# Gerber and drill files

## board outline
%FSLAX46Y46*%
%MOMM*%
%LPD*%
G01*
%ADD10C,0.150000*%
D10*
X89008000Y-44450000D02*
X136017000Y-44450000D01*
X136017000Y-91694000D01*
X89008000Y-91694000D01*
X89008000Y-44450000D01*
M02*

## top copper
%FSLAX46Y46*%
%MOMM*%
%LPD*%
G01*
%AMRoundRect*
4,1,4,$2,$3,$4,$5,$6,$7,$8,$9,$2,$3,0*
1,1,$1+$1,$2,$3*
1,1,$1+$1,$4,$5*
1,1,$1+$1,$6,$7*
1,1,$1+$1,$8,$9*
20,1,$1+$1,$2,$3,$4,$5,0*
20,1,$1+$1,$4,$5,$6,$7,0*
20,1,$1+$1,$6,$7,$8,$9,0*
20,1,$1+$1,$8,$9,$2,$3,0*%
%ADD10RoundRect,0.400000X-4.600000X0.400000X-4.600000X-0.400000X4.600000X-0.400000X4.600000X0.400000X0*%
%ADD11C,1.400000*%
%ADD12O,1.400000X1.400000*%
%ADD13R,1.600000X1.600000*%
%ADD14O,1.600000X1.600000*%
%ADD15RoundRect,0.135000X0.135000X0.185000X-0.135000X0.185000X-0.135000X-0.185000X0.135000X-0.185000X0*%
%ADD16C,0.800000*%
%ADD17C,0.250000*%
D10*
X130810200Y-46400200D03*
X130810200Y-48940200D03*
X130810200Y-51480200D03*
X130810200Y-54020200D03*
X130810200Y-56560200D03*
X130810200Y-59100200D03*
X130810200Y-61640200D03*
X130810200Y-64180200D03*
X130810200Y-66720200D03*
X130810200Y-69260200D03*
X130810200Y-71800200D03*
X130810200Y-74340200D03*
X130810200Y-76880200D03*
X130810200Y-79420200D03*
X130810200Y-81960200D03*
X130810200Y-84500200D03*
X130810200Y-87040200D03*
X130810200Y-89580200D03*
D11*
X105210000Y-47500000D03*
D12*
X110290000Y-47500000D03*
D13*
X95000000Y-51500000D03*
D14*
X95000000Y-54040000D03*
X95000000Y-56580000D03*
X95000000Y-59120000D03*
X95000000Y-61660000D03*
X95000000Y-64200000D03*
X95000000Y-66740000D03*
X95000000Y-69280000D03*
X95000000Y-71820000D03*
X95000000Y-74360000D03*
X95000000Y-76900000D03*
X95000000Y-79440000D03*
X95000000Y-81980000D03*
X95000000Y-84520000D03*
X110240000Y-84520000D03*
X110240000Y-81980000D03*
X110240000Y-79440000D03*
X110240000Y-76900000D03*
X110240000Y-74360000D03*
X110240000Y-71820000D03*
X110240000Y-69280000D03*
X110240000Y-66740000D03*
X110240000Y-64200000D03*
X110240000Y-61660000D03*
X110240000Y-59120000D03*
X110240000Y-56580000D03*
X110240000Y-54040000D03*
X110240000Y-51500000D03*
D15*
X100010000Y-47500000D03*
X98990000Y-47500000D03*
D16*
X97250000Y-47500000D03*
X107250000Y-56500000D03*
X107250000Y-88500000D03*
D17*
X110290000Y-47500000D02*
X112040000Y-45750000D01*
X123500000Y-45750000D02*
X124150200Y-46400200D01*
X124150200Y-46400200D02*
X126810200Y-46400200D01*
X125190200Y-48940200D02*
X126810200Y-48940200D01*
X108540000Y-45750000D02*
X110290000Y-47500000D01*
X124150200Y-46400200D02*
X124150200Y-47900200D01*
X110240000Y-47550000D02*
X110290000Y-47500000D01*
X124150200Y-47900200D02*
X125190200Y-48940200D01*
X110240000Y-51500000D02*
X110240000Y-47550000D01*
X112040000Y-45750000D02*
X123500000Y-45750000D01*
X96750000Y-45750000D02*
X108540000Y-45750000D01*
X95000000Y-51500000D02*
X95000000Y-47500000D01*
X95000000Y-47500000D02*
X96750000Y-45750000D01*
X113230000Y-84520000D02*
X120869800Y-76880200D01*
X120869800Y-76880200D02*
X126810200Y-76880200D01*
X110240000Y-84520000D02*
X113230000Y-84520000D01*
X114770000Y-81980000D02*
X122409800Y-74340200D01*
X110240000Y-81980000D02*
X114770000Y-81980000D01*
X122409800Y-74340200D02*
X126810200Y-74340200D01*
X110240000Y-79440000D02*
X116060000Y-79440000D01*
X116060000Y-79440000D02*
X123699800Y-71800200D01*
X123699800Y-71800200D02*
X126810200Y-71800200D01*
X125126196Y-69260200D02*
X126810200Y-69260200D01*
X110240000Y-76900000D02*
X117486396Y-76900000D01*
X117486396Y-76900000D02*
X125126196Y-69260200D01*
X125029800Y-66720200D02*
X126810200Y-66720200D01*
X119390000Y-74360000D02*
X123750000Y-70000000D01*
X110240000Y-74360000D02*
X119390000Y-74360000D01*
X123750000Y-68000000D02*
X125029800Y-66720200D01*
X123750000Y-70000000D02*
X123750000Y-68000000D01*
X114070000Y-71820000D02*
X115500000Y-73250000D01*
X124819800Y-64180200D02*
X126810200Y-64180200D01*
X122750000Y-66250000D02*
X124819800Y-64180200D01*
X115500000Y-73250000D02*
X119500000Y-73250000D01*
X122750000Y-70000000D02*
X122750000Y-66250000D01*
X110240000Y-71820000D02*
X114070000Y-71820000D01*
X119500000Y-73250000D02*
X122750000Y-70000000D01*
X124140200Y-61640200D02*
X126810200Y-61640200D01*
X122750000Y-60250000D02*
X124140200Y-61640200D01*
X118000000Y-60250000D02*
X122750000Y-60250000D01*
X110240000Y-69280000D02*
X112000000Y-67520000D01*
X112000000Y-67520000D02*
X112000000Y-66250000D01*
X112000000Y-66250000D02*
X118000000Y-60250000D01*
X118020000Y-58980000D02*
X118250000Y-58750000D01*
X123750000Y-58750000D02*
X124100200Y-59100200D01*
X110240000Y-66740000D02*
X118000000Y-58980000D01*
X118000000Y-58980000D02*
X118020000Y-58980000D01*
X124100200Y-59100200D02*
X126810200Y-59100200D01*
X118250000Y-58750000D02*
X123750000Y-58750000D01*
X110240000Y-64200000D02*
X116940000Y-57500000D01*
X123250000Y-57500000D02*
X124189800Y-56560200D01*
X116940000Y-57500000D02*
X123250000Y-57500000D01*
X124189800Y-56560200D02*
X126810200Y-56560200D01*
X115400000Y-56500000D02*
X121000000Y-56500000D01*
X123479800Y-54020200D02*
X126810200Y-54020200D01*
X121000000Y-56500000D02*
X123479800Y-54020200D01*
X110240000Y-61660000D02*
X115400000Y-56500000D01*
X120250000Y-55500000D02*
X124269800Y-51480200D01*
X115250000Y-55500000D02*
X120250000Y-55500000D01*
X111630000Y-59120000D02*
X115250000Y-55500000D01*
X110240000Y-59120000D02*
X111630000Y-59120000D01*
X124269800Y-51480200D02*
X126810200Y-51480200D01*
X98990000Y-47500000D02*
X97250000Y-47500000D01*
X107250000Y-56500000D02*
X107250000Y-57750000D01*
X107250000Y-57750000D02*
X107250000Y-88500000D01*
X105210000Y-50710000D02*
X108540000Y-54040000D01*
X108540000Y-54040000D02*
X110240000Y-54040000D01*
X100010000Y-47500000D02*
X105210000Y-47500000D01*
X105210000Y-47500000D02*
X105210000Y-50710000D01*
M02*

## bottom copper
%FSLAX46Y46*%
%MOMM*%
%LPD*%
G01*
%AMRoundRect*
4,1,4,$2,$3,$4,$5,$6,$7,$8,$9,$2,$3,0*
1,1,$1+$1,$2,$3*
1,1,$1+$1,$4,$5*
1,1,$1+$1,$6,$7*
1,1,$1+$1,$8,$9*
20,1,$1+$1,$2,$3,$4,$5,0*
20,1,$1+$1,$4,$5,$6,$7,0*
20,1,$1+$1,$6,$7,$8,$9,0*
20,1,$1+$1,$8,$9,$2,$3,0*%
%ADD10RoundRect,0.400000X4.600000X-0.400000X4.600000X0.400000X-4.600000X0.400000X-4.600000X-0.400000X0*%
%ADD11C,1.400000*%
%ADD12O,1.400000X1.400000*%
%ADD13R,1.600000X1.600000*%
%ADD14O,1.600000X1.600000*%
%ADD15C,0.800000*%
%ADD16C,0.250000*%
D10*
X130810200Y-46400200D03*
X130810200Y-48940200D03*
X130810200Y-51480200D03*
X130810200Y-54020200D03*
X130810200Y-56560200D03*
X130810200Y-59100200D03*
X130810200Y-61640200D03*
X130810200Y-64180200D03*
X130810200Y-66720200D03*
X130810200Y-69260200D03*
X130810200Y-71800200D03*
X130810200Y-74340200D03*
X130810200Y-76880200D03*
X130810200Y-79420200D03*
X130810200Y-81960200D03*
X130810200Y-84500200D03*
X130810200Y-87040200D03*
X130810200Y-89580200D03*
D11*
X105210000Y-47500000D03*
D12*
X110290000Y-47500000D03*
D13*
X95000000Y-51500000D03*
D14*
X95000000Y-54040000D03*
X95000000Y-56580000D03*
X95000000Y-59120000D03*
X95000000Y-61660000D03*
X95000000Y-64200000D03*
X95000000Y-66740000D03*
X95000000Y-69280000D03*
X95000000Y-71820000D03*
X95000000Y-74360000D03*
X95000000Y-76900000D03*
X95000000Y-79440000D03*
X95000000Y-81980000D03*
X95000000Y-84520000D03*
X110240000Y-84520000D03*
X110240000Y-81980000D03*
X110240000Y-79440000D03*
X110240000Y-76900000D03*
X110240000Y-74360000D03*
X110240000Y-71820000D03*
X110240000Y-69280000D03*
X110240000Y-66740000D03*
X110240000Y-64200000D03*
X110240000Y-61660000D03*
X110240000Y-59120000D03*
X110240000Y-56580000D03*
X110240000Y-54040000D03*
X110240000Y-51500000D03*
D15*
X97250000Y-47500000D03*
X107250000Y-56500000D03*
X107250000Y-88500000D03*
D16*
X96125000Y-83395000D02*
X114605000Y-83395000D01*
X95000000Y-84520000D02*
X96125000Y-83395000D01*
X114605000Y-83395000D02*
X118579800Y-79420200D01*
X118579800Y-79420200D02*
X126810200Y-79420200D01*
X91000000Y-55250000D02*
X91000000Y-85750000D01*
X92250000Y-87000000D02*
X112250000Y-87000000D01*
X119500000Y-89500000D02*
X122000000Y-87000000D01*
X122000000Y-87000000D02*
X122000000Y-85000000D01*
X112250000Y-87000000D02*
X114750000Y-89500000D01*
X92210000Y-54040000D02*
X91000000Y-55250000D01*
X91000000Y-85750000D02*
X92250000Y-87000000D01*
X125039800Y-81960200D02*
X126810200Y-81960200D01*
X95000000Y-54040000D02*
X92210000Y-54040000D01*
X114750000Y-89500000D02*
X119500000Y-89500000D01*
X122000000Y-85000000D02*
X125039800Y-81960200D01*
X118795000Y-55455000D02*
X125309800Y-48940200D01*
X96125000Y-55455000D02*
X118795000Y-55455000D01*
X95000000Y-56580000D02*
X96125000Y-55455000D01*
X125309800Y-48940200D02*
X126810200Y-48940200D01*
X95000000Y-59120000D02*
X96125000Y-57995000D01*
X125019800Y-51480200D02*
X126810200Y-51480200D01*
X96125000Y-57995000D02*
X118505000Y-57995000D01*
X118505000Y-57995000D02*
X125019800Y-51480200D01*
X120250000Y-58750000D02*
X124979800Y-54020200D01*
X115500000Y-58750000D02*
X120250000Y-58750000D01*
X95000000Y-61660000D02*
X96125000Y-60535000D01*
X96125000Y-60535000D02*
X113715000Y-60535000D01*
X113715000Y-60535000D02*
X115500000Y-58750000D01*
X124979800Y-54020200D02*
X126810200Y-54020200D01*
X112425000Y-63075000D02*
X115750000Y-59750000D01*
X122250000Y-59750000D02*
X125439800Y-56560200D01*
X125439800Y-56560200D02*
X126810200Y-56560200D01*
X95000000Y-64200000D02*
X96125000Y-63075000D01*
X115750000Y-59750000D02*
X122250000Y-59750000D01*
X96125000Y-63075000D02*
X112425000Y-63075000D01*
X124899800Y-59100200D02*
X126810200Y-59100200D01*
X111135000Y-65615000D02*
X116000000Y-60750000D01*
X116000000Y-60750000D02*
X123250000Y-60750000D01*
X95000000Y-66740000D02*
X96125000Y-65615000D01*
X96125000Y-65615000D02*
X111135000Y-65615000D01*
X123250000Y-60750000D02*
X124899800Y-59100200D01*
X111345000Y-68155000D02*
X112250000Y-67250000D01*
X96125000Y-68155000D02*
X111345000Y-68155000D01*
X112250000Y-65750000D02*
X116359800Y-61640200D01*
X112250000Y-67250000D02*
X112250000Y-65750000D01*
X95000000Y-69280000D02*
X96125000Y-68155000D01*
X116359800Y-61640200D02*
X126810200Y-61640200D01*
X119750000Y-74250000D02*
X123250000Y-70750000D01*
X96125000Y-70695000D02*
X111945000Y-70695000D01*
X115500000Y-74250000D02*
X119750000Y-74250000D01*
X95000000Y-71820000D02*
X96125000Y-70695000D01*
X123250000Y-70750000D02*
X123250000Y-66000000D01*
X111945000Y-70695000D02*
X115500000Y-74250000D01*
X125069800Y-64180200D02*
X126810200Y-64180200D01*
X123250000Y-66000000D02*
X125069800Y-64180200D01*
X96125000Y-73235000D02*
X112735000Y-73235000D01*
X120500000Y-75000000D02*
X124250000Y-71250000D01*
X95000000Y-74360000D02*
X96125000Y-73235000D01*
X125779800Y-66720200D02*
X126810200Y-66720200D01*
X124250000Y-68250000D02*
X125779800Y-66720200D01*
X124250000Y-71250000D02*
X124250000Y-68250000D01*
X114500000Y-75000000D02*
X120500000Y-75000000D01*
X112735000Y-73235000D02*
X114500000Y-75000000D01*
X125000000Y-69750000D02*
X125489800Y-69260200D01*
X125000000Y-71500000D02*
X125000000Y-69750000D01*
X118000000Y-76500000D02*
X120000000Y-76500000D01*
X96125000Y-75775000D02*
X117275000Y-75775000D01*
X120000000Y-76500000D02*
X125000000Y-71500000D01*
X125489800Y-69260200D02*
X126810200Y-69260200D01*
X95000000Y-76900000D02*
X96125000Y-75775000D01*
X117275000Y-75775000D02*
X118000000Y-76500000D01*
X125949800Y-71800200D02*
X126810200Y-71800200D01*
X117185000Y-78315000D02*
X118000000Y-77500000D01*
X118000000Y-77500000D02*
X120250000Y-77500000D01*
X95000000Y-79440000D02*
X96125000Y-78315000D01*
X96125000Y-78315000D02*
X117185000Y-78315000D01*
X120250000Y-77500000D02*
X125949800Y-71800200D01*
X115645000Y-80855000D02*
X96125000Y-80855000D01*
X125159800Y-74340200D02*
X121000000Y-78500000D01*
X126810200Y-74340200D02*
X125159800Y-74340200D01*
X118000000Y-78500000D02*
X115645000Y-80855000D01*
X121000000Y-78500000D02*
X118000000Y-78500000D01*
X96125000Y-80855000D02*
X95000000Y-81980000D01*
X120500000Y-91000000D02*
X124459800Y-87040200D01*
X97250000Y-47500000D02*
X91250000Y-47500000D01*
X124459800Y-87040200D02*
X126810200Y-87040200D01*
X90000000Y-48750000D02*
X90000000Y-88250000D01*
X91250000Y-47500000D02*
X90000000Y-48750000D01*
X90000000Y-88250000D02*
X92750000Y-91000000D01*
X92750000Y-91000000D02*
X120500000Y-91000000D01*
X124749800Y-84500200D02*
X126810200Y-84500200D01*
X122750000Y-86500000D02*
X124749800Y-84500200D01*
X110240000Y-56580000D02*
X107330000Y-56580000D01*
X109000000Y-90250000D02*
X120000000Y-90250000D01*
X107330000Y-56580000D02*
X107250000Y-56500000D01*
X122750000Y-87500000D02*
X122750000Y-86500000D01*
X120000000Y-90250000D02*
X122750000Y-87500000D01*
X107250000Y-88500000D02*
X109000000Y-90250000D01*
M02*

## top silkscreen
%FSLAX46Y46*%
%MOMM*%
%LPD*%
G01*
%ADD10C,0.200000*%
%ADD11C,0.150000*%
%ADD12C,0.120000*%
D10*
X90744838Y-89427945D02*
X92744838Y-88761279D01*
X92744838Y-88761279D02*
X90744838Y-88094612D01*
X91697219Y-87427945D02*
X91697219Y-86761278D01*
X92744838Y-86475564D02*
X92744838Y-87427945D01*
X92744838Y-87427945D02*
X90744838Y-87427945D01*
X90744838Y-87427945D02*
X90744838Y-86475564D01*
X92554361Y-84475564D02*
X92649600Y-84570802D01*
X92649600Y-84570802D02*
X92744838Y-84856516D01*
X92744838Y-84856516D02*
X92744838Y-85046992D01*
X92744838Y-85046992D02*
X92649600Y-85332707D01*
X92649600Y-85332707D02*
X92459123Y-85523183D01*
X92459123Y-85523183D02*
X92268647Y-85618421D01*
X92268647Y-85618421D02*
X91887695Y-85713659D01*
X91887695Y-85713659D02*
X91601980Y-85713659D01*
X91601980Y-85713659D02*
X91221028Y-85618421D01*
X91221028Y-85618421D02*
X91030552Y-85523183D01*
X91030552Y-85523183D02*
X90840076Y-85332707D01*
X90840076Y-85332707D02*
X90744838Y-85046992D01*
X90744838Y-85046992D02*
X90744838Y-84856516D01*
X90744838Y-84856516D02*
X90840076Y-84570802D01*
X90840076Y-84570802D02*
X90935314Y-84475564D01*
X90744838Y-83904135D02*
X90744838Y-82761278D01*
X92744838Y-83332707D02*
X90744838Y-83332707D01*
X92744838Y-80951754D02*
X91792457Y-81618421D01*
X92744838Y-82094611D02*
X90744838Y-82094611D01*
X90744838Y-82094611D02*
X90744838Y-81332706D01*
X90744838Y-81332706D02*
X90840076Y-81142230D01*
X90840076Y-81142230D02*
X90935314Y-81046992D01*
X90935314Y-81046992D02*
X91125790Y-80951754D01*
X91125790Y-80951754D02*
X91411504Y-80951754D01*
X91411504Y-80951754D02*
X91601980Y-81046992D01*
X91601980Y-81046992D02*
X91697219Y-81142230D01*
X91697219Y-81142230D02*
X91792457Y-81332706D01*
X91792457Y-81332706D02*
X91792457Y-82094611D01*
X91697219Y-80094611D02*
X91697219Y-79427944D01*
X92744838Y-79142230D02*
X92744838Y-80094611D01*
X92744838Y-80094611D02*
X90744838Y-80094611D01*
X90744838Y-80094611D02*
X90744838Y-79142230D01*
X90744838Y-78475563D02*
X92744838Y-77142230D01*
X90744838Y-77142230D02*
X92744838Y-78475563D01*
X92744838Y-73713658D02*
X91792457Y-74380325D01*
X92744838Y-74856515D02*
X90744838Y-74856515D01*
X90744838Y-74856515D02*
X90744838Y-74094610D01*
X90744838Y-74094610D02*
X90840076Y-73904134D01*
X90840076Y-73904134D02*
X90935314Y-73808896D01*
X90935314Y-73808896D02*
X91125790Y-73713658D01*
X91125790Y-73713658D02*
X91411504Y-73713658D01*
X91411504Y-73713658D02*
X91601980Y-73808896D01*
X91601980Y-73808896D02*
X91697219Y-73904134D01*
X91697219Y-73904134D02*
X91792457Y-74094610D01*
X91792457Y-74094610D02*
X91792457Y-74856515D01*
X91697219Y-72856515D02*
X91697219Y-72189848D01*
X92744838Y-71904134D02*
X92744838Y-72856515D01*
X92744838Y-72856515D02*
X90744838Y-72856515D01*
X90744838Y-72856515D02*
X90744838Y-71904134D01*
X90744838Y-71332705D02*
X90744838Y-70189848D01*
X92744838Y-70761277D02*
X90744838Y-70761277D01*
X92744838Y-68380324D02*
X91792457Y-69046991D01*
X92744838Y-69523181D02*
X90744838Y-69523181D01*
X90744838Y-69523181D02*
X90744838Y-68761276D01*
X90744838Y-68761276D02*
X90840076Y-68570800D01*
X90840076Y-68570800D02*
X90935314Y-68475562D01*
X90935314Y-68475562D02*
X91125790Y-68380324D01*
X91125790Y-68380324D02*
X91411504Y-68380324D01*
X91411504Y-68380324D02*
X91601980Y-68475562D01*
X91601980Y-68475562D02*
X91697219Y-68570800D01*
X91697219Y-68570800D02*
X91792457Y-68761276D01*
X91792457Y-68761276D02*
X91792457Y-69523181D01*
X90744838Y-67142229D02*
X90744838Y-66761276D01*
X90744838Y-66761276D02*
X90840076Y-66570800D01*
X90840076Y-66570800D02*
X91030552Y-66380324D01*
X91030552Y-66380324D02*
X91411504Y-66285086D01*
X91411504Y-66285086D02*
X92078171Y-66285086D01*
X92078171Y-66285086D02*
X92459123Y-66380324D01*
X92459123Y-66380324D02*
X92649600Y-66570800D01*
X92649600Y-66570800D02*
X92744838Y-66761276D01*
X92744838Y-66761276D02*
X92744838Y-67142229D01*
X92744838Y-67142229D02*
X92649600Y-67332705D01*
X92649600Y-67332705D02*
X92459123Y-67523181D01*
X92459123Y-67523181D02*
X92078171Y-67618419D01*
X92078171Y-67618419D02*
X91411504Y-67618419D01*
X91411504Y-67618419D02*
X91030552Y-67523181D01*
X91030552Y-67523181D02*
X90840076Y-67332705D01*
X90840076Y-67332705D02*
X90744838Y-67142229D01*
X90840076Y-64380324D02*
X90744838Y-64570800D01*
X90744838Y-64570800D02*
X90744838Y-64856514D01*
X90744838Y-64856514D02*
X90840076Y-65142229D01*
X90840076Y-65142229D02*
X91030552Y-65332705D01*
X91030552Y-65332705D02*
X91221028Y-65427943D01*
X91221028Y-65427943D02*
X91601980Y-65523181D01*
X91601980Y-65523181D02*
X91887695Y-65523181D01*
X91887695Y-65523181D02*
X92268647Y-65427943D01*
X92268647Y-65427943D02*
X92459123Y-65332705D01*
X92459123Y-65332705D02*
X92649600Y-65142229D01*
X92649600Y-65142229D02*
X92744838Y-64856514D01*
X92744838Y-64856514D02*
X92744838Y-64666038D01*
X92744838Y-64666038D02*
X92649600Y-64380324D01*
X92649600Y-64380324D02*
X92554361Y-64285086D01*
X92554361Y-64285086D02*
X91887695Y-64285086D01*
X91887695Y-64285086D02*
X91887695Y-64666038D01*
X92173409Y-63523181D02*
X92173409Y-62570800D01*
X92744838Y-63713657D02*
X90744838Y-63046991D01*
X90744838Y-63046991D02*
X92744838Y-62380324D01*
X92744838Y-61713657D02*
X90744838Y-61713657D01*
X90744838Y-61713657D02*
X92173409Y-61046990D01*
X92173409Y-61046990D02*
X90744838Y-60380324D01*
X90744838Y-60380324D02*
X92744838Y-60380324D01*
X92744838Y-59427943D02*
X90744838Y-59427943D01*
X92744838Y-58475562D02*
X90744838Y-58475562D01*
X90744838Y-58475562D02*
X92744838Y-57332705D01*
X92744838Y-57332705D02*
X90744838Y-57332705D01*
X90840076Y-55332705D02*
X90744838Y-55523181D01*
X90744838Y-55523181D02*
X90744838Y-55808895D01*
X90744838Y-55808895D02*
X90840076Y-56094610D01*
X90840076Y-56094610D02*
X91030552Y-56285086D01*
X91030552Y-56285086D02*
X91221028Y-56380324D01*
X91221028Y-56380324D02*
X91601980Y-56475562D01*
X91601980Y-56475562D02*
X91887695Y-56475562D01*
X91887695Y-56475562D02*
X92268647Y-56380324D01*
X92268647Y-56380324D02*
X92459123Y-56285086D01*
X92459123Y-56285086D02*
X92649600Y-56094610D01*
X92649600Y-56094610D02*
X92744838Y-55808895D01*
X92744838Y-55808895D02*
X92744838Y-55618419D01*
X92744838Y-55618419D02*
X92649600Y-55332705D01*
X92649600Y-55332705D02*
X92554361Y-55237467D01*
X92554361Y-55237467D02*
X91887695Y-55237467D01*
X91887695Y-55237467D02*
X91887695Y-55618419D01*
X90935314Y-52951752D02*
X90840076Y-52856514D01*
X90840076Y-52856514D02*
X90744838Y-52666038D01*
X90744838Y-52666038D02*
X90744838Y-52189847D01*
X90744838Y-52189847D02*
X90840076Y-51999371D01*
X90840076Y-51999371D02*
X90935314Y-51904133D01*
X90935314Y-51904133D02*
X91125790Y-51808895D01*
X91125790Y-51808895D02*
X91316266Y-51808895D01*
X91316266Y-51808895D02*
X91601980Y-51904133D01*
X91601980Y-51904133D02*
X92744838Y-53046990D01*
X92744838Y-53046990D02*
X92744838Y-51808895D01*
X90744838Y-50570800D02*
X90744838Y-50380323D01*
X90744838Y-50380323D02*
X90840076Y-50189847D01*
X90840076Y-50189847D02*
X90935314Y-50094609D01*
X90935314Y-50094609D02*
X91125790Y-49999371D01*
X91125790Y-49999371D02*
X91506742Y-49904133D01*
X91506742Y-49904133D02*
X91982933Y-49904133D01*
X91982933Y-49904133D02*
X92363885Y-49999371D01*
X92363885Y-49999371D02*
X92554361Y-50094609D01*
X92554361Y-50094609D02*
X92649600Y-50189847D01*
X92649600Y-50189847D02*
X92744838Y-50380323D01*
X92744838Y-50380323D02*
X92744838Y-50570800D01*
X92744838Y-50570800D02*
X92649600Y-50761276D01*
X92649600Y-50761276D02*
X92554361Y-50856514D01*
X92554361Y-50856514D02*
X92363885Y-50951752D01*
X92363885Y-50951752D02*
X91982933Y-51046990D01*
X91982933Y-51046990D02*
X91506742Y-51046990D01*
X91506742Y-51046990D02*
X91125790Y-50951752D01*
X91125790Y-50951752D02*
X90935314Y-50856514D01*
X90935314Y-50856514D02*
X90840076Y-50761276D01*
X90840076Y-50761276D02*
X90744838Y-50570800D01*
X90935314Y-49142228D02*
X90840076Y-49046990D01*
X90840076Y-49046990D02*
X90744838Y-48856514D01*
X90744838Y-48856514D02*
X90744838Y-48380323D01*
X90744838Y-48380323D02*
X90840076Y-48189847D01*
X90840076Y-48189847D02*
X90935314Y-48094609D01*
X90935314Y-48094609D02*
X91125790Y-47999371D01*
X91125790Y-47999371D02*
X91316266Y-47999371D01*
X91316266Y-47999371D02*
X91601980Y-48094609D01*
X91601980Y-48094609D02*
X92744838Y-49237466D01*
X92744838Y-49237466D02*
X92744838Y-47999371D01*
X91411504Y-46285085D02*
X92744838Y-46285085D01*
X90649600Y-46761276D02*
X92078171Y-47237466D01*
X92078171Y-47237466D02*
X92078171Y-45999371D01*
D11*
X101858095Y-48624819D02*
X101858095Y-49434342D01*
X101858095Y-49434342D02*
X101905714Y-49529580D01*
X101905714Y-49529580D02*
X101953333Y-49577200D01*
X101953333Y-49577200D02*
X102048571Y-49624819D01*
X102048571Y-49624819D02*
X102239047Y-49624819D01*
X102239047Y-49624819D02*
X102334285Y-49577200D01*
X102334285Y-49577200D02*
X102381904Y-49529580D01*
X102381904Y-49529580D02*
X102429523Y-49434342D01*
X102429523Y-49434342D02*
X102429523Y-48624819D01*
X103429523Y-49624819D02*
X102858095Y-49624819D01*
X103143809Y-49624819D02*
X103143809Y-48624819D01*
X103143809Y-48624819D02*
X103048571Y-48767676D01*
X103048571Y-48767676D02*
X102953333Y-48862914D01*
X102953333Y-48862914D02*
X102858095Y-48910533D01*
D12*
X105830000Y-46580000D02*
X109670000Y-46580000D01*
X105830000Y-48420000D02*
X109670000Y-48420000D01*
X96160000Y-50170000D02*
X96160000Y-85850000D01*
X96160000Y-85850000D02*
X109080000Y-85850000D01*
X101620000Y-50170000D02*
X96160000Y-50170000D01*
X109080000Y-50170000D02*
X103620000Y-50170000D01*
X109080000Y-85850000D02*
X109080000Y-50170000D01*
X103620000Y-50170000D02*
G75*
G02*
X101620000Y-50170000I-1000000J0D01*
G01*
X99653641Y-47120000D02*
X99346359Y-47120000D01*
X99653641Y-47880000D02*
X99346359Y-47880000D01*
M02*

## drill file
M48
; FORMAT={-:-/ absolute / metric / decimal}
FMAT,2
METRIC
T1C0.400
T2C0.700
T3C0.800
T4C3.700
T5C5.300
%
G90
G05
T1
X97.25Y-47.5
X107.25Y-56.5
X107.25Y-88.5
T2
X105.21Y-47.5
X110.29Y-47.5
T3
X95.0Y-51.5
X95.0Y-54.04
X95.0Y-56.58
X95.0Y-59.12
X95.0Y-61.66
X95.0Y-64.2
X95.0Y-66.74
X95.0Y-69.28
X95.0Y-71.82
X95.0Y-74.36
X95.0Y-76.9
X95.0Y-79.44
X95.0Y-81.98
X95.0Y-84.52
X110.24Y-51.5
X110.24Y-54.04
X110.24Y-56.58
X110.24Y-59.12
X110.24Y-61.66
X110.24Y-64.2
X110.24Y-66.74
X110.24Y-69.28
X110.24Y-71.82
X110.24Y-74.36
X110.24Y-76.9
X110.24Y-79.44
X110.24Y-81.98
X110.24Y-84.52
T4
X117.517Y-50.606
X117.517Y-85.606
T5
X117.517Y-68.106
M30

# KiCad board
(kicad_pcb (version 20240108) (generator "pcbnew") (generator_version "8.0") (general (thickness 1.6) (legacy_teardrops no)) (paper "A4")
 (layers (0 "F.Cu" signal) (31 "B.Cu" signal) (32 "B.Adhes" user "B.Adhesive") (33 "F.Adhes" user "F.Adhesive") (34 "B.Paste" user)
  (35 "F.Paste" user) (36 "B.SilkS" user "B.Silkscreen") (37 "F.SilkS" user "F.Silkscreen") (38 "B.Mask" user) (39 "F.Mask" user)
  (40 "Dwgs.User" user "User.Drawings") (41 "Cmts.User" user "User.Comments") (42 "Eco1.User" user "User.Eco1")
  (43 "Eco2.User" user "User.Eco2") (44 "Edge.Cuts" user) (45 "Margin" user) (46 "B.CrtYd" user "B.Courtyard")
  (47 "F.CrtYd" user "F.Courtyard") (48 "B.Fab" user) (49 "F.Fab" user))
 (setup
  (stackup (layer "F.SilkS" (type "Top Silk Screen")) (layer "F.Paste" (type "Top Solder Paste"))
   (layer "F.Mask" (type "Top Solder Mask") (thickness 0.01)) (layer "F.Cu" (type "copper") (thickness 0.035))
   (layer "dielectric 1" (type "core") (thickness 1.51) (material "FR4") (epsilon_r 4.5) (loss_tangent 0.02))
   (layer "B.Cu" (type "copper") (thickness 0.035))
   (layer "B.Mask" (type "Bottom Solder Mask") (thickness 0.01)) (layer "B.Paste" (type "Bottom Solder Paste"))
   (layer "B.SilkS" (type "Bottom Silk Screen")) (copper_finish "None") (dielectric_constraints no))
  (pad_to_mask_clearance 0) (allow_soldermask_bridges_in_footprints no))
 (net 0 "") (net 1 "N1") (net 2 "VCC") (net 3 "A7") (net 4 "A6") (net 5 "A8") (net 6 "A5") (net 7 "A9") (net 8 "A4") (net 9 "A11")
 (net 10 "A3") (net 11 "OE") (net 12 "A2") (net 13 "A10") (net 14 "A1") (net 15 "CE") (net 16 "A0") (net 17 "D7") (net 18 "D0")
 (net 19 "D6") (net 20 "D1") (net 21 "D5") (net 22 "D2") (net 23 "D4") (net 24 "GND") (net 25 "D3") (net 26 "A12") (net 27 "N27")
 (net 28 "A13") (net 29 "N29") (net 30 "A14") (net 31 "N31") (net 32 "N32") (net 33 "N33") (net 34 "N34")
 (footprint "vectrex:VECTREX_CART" (layer "F.Cu") (at 130.8102 67.9902 -90)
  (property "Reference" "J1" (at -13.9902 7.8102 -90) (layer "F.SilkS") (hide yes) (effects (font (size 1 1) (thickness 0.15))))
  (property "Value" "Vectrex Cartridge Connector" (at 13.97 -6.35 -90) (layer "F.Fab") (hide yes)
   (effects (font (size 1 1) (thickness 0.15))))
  (pad "1" connect roundrect (at -21.59 4 90) (size 1.6 10) (drill (offset 0 4)) (layers "B.Cu" "B.Mask") (roundrect_rratio 0.25)
   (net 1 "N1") (zone_connect 2))
  (pad "2" connect roundrect (at -21.59 4 270) (size 1.6 10) (drill (offset 0 -4)) (layers "F.Cu" "F.Mask") (roundrect_rratio 0.25)
   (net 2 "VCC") (zone_connect 2))
  (pad "3" connect roundrect (at -19.05 4 90) (size 1.6 10) (drill (offset 0 4)) (layers "B.Cu" "B.Mask") (roundrect_rratio 0.25)
   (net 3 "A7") (zone_connect 2))
  (pad "4" connect roundrect (at -19.05 4 270) (size 1.6 10) (drill (offset 0 -4)) (layers "F.Cu" "F.Mask") (roundrect_rratio 0.25)
   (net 2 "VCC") (zone_connect 2))
  (pad "5" connect roundrect (at -16.51 4 90) (size 1.6 10) (drill (offset 0 4)) (layers "B.Cu" "B.Mask") (roundrect_rratio 0.25)
   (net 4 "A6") (zone_connect 2))
  (pad "6" connect roundrect (at -16.51 4 270) (size 1.6 10) (drill (offset 0 -4)) (layers "F.Cu" "F.Mask") (roundrect_rratio 0.25)
   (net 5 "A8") (zone_connect 2))
  (pad "7" connect roundrect (at -13.97 4 90) (size 1.6 10) (drill (offset 0 4)) (layers "B.Cu" "B.Mask") (roundrect_rratio 0.25)
   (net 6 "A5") (zone_connect 2))
  (pad "8" connect roundrect (at -13.97 4 270) (size 1.6 10) (drill (offset 0 -4)) (layers "F.Cu" "F.Mask") (roundrect_rratio 0.25)
   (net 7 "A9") (zone_connect 2))
  (pad "9" connect roundrect (at -11.43 4 90) (size 1.6 10) (drill (offset 0 4)) (layers "B.Cu" "B.Mask") (roundrect_rratio 0.25)
   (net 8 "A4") (zone_connect 2))
  (pad "10" connect roundrect (at -11.43 4 270) (size 1.6 10) (drill (offset 0 -4)) (layers "F.Cu" "F.Mask") (roundrect_rratio 0.25)
   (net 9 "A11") (zone_connect 2))
  (pad "11" connect roundrect (at -8.89 4 90) (size 1.6 10) (drill (offset 0 4)) (layers "B.Cu" "B.Mask") (roundrect_rratio 0.25)
   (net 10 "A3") (zone_connect 2))
  (pad "12" connect roundrect (at -8.89 4 270) (size 1.6 10) (drill (offset 0 -4)) (layers "F.Cu" "F.Mask") (roundrect_rratio 0.25)
   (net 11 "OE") (zone_connect 2))
  (pad "13" connect roundrect (at -6.35 4 90) (size 1.6 10) (drill (offset 0 4)) (layers "B.Cu" "B.Mask") (roundrect_rratio 0.25)
   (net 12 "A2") (zone_connect 2))
  (pad "14" connect roundrect (at -6.35 4 270) (size 1.6 10) (drill (offset 0 -4)) (layers "F.Cu" "F.Mask") (roundrect_rratio 0.25)
   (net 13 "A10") (zone_connect 2))
  (pad "15" connect roundrect (at -3.81 4 90) (size 1.6 10) (drill (offset 0 4)) (layers "B.Cu" "B.Mask") (roundrect_rratio 0.25)
   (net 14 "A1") (zone_connect 2))
  (pad "16" connect roundrect (at -3.81 4 270) (size 1.6 10) (drill (offset 0 -4)) (layers "F.Cu" "F.Mask") (roundrect_rratio 0.25)
   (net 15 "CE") (zone_connect 2))
  (pad "17" connect roundrect (at -1.27 4 90) (size 1.6 10) (drill (offset 0 4)) (layers "B.Cu" "B.Mask") (roundrect_rratio 0.25)
   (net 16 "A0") (zone_connect 2))
  (pad "18" connect roundrect (at -1.27 4 270) (size 1.6 10) (drill (offset 0 -4)) (layers "F.Cu" "F.Mask") (roundrect_rratio 0.25)
   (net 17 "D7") (zone_connect 2))
  (pad "19" connect roundrect (at 1.27 4 90) (size 1.6 10) (drill (offset 0 4)) (layers "B.Cu" "B.Mask") (roundrect_rratio 0.25)
   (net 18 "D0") (zone_connect 2))
  (pad "20" connect roundrect (at 1.27 4 270) (size 1.6 10) (drill (offset 0 -4)) (layers "F.Cu" "F.Mask") (roundrect_rratio 0.25)
   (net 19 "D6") (zone_connect 2))
  (pad "21" connect roundrect (at 3.81 4 90) (size 1.6 10) (drill (offset 0 4)) (layers "B.Cu" "B.Mask") (roundrect_rratio 0.25)
   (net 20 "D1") (zone_connect 2))
  (pad "22" connect roundrect (at 3.81 4 270) (size 1.6 10) (drill (offset 0 -4)) (layers "F.Cu" "F.Mask") (roundrect_rratio 0.25)
   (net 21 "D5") (zone_connect 2))
  (pad "23" connect roundrect (at 6.35 4 90) (size 1.6 10) (drill (offset 0 4)) (layers "B.Cu" "B.Mask") (roundrect_rratio 0.25)
   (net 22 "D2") (zone_connect 2))
  (pad "24" connect roundrect (at 6.35 4 270) (size 1.6 10) (drill (offset 0 -4)) (layers "F.Cu" "F.Mask") (roundrect_rratio 0.25)
   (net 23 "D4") (zone_connect 2))
  (pad "25" connect roundrect (at 8.89 4 90) (size 1.6 10) (drill (offset 0 4)) (layers "B.Cu" "B.Mask") (roundrect_rratio 0.25)
   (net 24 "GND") (zone_connect 2))
  (pad "26" connect roundrect (at 8.89 4 270) (size 1.6 10) (drill (offset 0 -4)) (layers "F.Cu" "F.Mask") (roundrect_rratio 0.25)
   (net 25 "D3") (zone_connect 2))
  (pad "27" connect roundrect (at 11.43 4 90) (size 1.6 10) (drill (offset 0 4)) (layers "B.Cu" "B.Mask") (roundrect_rratio 0.25)
   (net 24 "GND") (zone_connect 2))
  (pad "28" connect roundrect (at 11.43 4 270) (size 1.6 10) (drill (offset 0 -4)) (layers "F.Cu" "F.Mask") (roundrect_rratio 0.25)
   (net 24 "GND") (zone_connect 2))
  (pad "29" connect roundrect (at 13.97 4 90) (size 1.6 10) (drill (offset 0 4)) (layers "B.Cu" "B.Mask") (roundrect_rratio 0.25)
   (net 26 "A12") (zone_connect 2))
  (pad "30" connect roundrect (at 13.97 4 270) (size 1.6 10) (drill (offset 0 -4)) (layers "F.Cu" "F.Mask") (roundrect_rratio 0.25)
   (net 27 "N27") (zone_connect 2))
  (pad "31" connect roundrect (at 16.51 4 90) (size 1.6 10) (drill (offset 0 4)) (layers "B.Cu" "B.Mask") (roundrect_rratio 0.25)
   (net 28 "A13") (zone_connect 2))
  (pad "32" connect roundrect (at 16.51 4 270) (size 1.6 10) (drill (offset 0 -4)) (layers "F.Cu" "F.Mask") (roundrect_rratio 0.25)
   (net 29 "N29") (zone_connect 2))
  (pad "33" connect roundrect (at 19.05 4 90) (size 1.6 10) (drill (offset 0 4)) (layers "B.Cu" "B.Mask") (roundrect_rratio 0.25)
   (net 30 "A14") (zone_connect 2))
  (pad "34" connect roundrect (at 19.05 4 270) (size 1.6 10) (drill (offset 0 -4)) (layers "F.Cu" "F.Mask") (roundrect_rratio 0.25)
   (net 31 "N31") (zone_connect 2))
  (pad "35" connect roundrect (at 21.59 4 90) (size 1.6 10) (drill (offset 0 4)) (layers "B.Cu" "B.Mask") (roundrect_rratio 0.25)
   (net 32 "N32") (zone_connect 2))
  (pad "36" connect roundrect (at 21.59 4 270) (size 1.6 10) (drill (offset 0 -4)) (layers "F.Cu" "F.Mask") (roundrect_rratio 0.25)
   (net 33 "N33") (zone_connect 2)))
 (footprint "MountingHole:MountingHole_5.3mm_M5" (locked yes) (layer "F.Cu") (at 117.5172 68.1056)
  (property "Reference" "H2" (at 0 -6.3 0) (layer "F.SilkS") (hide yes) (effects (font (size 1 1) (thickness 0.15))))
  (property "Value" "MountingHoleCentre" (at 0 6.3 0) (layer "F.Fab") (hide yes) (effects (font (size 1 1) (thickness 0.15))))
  (pad "" np_thru_hole circle (at 0 0) (size 5.3 5.3) (drill 5.3) (layers "*.Cu" "*.Mask")))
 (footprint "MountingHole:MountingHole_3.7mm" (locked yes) (layer "F.Cu") (at 117.5172 50.6056)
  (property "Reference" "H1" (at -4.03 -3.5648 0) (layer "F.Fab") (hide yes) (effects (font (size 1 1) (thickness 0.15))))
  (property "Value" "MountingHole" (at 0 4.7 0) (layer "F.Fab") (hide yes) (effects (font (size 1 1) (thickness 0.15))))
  (pad "" np_thru_hole circle (at 0 0) (size 3.7 3.7) (drill 3.7) (layers "*.Cu" "*.Mask")))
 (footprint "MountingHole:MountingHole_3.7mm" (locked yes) (layer "F.Cu") (at 117.5172 85.6056)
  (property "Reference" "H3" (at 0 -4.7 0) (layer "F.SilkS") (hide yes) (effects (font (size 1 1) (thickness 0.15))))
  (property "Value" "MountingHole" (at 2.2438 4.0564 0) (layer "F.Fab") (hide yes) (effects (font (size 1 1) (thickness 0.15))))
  (pad "" np_thru_hole circle (at 0 0) (size 3.7 3.7) (drill 3.7) (layers "*.Cu" "*.Mask")))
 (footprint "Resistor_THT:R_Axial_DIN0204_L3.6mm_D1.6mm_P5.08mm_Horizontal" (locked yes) (layer "F.Cu") (at 105.21 47.5)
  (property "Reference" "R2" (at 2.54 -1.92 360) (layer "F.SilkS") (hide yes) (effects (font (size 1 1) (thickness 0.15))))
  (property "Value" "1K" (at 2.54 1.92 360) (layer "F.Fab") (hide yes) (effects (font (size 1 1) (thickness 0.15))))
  (fp_line (start 0.62 -0.92) (end 4.46 -0.92) (stroke (width 0.12) (type solid)) (layer "F.SilkS"))
  (fp_line (start 0.62 0.92) (end 4.46 0.92) (stroke (width 0.12) (type solid)) (layer "F.SilkS"))
  (pad "1" thru_hole circle (at 0 0) (size 1.4 1.4) (drill 0.7) (layers "*.Cu" "*.Mask") (remove_unused_layers no) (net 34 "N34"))
  (pad "2" thru_hole oval (at 5.08 0) (size 1.4 1.4) (drill 0.7) (layers "*.Cu" "*.Mask") (remove_unused_layers no) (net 2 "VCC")))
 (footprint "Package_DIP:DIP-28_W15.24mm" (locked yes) (layer "F.Cu") (at 95 51.5)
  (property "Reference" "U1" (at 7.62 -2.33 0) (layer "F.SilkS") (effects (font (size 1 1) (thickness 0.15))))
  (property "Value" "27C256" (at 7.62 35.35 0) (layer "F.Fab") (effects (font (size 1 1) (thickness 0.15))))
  (fp_line (start 1.16 -1.33) (end 1.16 34.35) (stroke (width 0.12) (type solid)) (layer "F.SilkS"))
  (fp_line (start 1.16 34.35) (end 14.08 34.35) (stroke (width 0.12) (type solid)) (layer "F.SilkS"))
  (fp_line (start 6.62 -1.33) (end 1.16 -1.33) (stroke (width 0.12) (type solid)) (layer "F.SilkS"))
  (fp_line (start 14.08 -1.33) (end 8.62 -1.33) (stroke (width 0.12) (type solid)) (layer "F.SilkS"))
  (fp_line (start 14.08 34.35) (end 14.08 -1.33) (stroke (width 0.12) (type solid)) (layer "F.SilkS"))
  (fp_arc (start 8.62 -1.33) (mid 7.62 -0.33) (end 6.62 -1.33) (stroke (width 0.12) (type solid)) (layer "F.SilkS"))
  (pad "1" thru_hole rect (at 0 0) (size 1.6 1.6) (drill 0.8) (layers "*.Cu" "*.Mask") (remove_unused_layers no) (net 2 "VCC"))
  (pad "2" thru_hole oval (at 0 2.54) (size 1.6 1.6) (drill 0.8) (layers "*.Cu" "*.Mask") (remove_unused_layers no) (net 26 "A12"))
  (pad "3" thru_hole oval (at 0 5.08) (size 1.6 1.6) (drill 0.8) (layers "*.Cu" "*.Mask") (remove_unused_layers no) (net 3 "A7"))
  (pad "4" thru_hole oval (at 0 7.62) (size 1.6 1.6) (drill 0.8) (layers "*.Cu" "*.Mask") (remove_unused_layers no) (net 4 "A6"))
  (pad "5" thru_hole oval (at 0 10.16) (size 1.6 1.6) (drill 0.8) (layers "*.Cu" "*.Mask") (remove_unused_layers no) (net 6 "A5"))
  (pad "6" thru_hole oval (at 0 12.7) (size 1.6 1.6) (drill 0.8) (layers "*.Cu" "*.Mask") (remove_unused_layers no) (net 8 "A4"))
  (pad "7" thru_hole oval (at 0 15.24) (size 1.6 1.6) (drill 0.8) (layers "*.Cu" "*.Mask") (remove_unused_layers no) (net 10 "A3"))
  (pad "8" thru_hole oval (at 0 17.78) (size 1.6 1.6) (drill 0.8) (layers "*.Cu" "*.Mask") (remove_unused_layers no) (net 12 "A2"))
  (pad "9" thru_hole oval (at 0 20.32) (size 1.6 1.6) (drill 0.8) (layers "*.Cu" "*.Mask") (remove_unused_layers no) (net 14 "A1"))
  (pad "10" thru_hole oval (at 0 22.86) (size 1.6 1.6) (drill 0.8) (layers "*.Cu" "*.Mask") (remove_unused_layers no) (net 16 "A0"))
  (pad "11" thru_hole oval (at 0 25.4) (size 1.6 1.6) (drill 0.8) (layers "*.Cu" "*.Mask") (remove_unused_layers no) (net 18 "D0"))
  (pad "12" thru_hole oval (at 0 27.94) (size 1.6 1.6) (drill 0.8) (layers "*.Cu" "*.Mask") (remove_unused_layers no) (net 20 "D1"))
  (pad "13" thru_hole oval (at 0 30.48) (size 1.6 1.6) (drill 0.8) (layers "*.Cu" "*.Mask") (remove_unused_layers no) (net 22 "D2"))
  (pad "14" thru_hole oval (at 0 33.02) (size 1.6 1.6) (drill 0.8) (layers "*.Cu" "*.Mask") (remove_unused_layers no) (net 24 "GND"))
  (pad "15" thru_hole oval (at 15.24 33.02) (size 1.6 1.6) (drill 0.8) (layers "*.Cu" "*.Mask") (remove_unused_layers no) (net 25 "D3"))
  (pad "16" thru_hole oval (at 15.24 30.48) (size 1.6 1.6) (drill 0.8) (layers "*.Cu" "*.Mask") (remove_unused_layers no) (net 23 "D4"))
  (pad "17" thru_hole oval (at 15.24 27.94) (size 1.6 1.6) (drill 0.8) (layers "*.Cu" "*.Mask") (remove_unused_layers no) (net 21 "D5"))
  (pad "18" thru_hole oval (at 15.24 25.4) (size 1.6 1.6) (drill 0.8) (layers "*.Cu" "*.Mask") (remove_unused_layers no) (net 19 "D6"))
  (pad "19" thru_hole oval (at 15.24 22.86) (size 1.6 1.6) (drill 0.8) (layers "*.Cu" "*.Mask") (remove_unused_layers no) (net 17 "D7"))
  (pad "20" thru_hole oval (at 15.24 20.32) (size 1.6 1.6) (drill 0.8) (layers "*.Cu" "*.Mask") (remove_unused_layers no) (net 15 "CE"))
  (pad "21" thru_hole oval (at 15.24 17.78) (size 1.6 1.6) (drill 0.8) (layers "*.Cu" "*.Mask") (remove_unused_layers no) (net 13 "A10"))
  (pad "22" thru_hole oval (at 15.24 15.24) (size 1.6 1.6) (drill 0.8) (layers "*.Cu" "*.Mask") (remove_unused_layers no) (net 11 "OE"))
  (pad "23" thru_hole oval (at 15.24 12.7) (size 1.6 1.6) (drill 0.8) (layers "*.Cu" "*.Mask") (remove_unused_layers no) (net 9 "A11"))
  (pad "24" thru_hole oval (at 15.24 10.16) (size 1.6 1.6) (drill 0.8) (layers "*.Cu" "*.Mask") (remove_unused_layers no) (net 7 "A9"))
  (pad "25" thru_hole oval (at 15.24 7.62) (size 1.6 1.6) (drill 0.8) (layers "*.Cu" "*.Mask") (remove_unused_layers no) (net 5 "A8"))
  (pad "26" thru_hole oval (at 15.24 5.08) (size 1.6 1.6) (drill 0.8) (layers "*.Cu" "*.Mask") (remove_unused_layers no) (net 28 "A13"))
  (pad "27" thru_hole oval (at 15.24 2.54) (size 1.6 1.6) (drill 0.8) (layers "*.Cu" "*.Mask") (remove_unused_layers no) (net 34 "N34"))
  (pad "28" thru_hole oval (at 15.24 0) (size 1.6 1.6) (drill 0.8) (layers "*.Cu" "*.Mask") (remove_unused_layers no) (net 2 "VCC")))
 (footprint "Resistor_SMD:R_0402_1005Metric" (layer "F.Cu") (at 99.5 47.5 180)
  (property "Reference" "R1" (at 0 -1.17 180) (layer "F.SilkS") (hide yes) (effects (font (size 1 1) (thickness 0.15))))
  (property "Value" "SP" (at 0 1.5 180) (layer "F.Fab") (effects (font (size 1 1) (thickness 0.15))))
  (fp_line (start -0.153641 0.38) (end 0.153641 0.38) (stroke (width 0.12) (type solid)) (layer "F.SilkS"))
  (fp_line (start -0.153641 -0.38) (end 0.153641 -0.38) (stroke (width 0.12) (type solid)) (layer "F.SilkS"))
  (pad "1" smd roundrect (at -0.51 0 180) (size 0.54 0.64) (layers "F.Cu" "F.Paste" "F.Mask") (roundrect_rratio 0.25) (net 34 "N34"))
  (pad "2" smd roundrect (at 0.51 0 180) (size 0.54 0.64) (layers "F.Cu" "F.Paste" "F.Mask") (roundrect_rratio 0.25) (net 30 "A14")))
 (gr_rect (start 89.008 44.45) (end 136.017 91.694) (stroke (width 0.15) (type solid)) (fill none) (layer "Edge.Cuts"))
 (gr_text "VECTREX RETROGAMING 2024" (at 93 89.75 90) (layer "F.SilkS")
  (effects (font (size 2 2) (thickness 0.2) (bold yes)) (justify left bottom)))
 (segment (start 96.125 83.395) (end 114.605 83.395) (width 0.25) (layer "B.Cu") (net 24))
 (segment (start 95 84.52) (end 96.125 83.395) (width 0.25) (layer "B.Cu") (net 24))
 (segment (start 114.605 83.395) (end 118.5798 79.4202) (width 0.25) (layer "B.Cu") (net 24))
 (segment (start 118.5798 79.4202) (end 126.8102 79.4202) (width 0.25) (layer "B.Cu") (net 24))
 (segment (start 110.29 47.5) (end 112.04 45.75) (width 0.25) (layer "F.Cu") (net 2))
 (segment (start 123.5 45.75) (end 124.1502 46.4002) (width 0.25) (layer "F.Cu") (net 2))
 (segment (start 124.1502 46.4002) (end 126.8102 46.4002) (width 0.25) (layer "F.Cu") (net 2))
 (segment (start 125.1902 48.9402) (end 126.8102 48.9402) (width 0.25) (layer "F.Cu") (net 2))
 (segment (start 108.54 45.75) (end 110.29 47.5) (width 0.25) (layer "F.Cu") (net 2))
 (segment (start 124.1502 46.4002) (end 124.1502 47.9002) (width 0.25) (layer "F.Cu") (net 2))
 (segment (start 110.24 47.55) (end 110.29 47.5) (width 0.25) (layer "F.Cu") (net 2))
 (segment (start 124.1502 47.9002) (end 125.1902 48.9402) (width 0.25) (layer "F.Cu") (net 2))
 (segment (start 110.24 51.5) (end 110.24 47.55) (width 0.25) (layer "F.Cu") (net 2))
 (segment (start 112.04 45.75) (end 123.5 45.75) (width 0.25) (layer "F.Cu") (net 2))
 (segment (start 96.75 45.75) (end 108.54 45.75) (width 0.25) (layer "F.Cu") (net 2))
 (segment (start 95 51.5) (end 95 47.5) (width 0.25) (layer "F.Cu") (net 2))
 (segment (start 95 47.5) (end 96.75 45.75) (width 0.25) (layer "F.Cu") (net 2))
 (segment (start 113.23 84.52) (end 120.8698 76.8802) (width 0.25) (layer "F.Cu") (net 25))
 (segment (start 120.8698 76.8802) (end 126.8102 76.8802) (width 0.25) (layer "F.Cu") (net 25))
 (segment (start 110.24 84.52) (end 113.23 84.52) (width 0.25) (layer "F.Cu") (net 25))
 (segment (start 114.77 81.98) (end 122.4098 74.3402) (width 0.25) (layer "F.Cu") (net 23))
 (segment (start 110.24 81.98) (end 114.77 81.98) (width 0.25) (layer "F.Cu") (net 23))
 (segment (start 122.4098 74.3402) (end 126.8102 74.3402) (width 0.25) (layer "F.Cu") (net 23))
 (segment (start 110.24 79.44) (end 116.06 79.44) (width 0.25) (layer "F.Cu") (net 21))
 (segment (start 116.06 79.44) (end 123.6998 71.8002) (width 0.25) (layer "F.Cu") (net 21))
 (segment (start 123.6998 71.8002) (end 126.8102 71.8002) (width 0.25) (layer "F.Cu") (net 21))
 (segment (start 91 55.25) (end 91 85.75) (width 0.25) (layer "B.Cu") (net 26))
 (segment (start 92.25 87) (end 112.25 87) (width 0.25) (layer "B.Cu") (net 26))
 (segment (start 119.5 89.5) (end 122 87) (width 0.25) (layer "B.Cu") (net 26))
 (segment (start 122 87) (end 122 85) (width 0.25) (layer "B.Cu") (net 26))
 (segment (start 112.25 87) (end 114.75 89.5) (width 0.25) (layer "B.Cu") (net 26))
 (segment (start 92.21 54.04) (end 91 55.25) (width 0.25) (layer "B.Cu") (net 26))
 (segment (start 91 85.75) (end 92.25 87) (width 0.25) (layer "B.Cu") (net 26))
 (segment (start 125.0398 81.9602) (end 126.8102 81.9602) (width 0.25) (layer "B.Cu") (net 26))
 (segment (start 95 54.04) (end 92.21 54.04) (width 0.25) (layer "B.Cu") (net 26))
 (segment (start 114.75 89.5) (end 119.5 89.5) (width 0.25) (layer "B.Cu") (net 26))
 (segment (start 122 85) (end 125.0398 81.9602) (width 0.25) (layer "B.Cu") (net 26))
 (segment (start 125.126196 69.2602) (end 126.8102 69.2602) (width 0.25) (layer "F.Cu") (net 19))
 (segment (start 110.24 76.9) (end 117.486396 76.9) (width 0.25) (layer "F.Cu") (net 19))
 (segment (start 117.486396 76.9) (end 125.126196 69.2602) (width 0.25) (layer "F.Cu") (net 19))
 (segment (start 118.795 55.455) (end 125.3098 48.9402) (width 0.25) (layer "B.Cu") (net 3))
 (segment (start 96.125 55.455) (end 118.795 55.455) (width 0.25) (layer "B.Cu") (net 3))
 (segment (start 95 56.58) (end 96.125 55.455) (width 0.25) (layer "B.Cu") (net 3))
 (segment (start 125.3098 48.9402) (end 126.8102 48.9402) (width 0.25) (layer "B.Cu") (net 3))
 (segment (start 125.0298 66.7202) (end 126.8102 66.7202) (width 0.25) (layer "F.Cu") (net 17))
 (segment (start 119.39 74.36) (end 123.75 70) (width 0.25) (layer "F.Cu") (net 17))
 (segment (start 110.24 74.36) (end 119.39 74.36) (width 0.25) (layer "F.Cu") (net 17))
 (segment (start 123.75 68) (end 125.0298 66.7202) (width 0.25) (layer "F.Cu") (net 17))
 (segment (start 123.75 70) (end 123.75 68) (width 0.25) (layer "F.Cu") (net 17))
 (segment (start 95 59.12) (end 96.125 57.995) (width 0.25) (layer "B.Cu") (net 4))
 (segment (start 125.0198 51.4802) (end 126.8102 51.4802) (width 0.25) (layer "B.Cu") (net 4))
 (segment (start 96.125 57.995) (end 118.505 57.995) (width 0.25) (layer "B.Cu") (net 4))
 (segment (start 118.505 57.995) (end 125.0198 51.4802) (width 0.25) (layer "B.Cu") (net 4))
 (segment (start 114.07 71.82) (end 115.5 73.25) (width 0.25) (layer "F.Cu") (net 15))
 (segment (start 124.8198 64.1802) (end 126.8102 64.1802) (width 0.25) (layer "F.Cu") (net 15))
 (segment (start 122.75 66.25) (end 124.8198 64.1802) (width 0.25) (layer "F.Cu") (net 15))
 (segment (start 115.5 73.25) (end 119.5 73.25) (width 0.25) (layer "F.Cu") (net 15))
 (segment (start 122.75 70) (end 122.75 66.25) (width 0.25) (layer "F.Cu") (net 15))
 (segment (start 110.24 71.82) (end 114.07 71.82) (width 0.25) (layer "F.Cu") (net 15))
 (segment (start 119.5 73.25) (end 122.75 70) (width 0.25) (layer "F.Cu") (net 15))
 (segment (start 120.25 58.75) (end 124.9798 54.0202) (width 0.25) (layer "B.Cu") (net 6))
 (segment (start 115.5 58.75) (end 120.25 58.75) (width 0.25) (layer "B.Cu") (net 6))
 (segment (start 95 61.66) (end 96.125 60.535) (width 0.25) (layer "B.Cu") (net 6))
 (segment (start 96.125 60.535) (end 113.715 60.535) (width 0.25) (layer "B.Cu") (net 6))
 (segment (start 113.715 60.535) (end 115.5 58.75) (width 0.25) (layer "B.Cu") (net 6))
 (segment (start 124.9798 54.0202) (end 126.8102 54.0202) (width 0.25) (layer "B.Cu") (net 6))
 (segment (start 124.1402 61.6402) (end 126.8102 61.6402) (width 0.25) (layer "F.Cu") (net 13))
 (segment (start 122.75 60.25) (end 124.1402 61.6402) (width 0.25) (layer "F.Cu") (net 13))
 (segment (start 118 60.25) (end 122.75 60.25) (width 0.25) (layer "F.Cu") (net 13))
 (segment (start 110.24 69.28) (end 112 67.52) (width 0.25) (layer "F.Cu") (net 13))
 (segment (start 112 67.52) (end 112 66.25) (width 0.25) (layer "F.Cu") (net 13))
 (segment (start 112 66.25) (end 118 60.25) (width 0.25) (layer "F.Cu") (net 13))
 (segment (start 112.425 63.075) (end 115.75 59.75) (width 0.25) (layer "B.Cu") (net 8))
 (segment (start 122.25 59.75) (end 125.4398 56.5602) (width 0.25) (layer "B.Cu") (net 8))
 (segment (start 125.4398 56.5602) (end 126.8102 56.5602) (width 0.25) (layer "B.Cu") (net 8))
 (segment (start 95 64.2) (end 96.125 63.075) (width 0.25) (layer "B.Cu") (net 8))
 (segment (start 115.75 59.75) (end 122.25 59.75) (width 0.25) (layer "B.Cu") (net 8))
 (segment (start 96.125 63.075) (end 112.425 63.075) (width 0.25) (layer "B.Cu") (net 8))
 (segment (start 118.02 58.98) (end 118.25 58.75) (width 0.25) (layer "F.Cu") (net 11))
 (segment (start 123.75 58.75) (end 124.1002 59.1002) (width 0.25) (layer "F.Cu") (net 11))
 (segment (start 110.24 66.74) (end 118 58.98) (width 0.25) (layer "F.Cu") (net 11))
 (segment (start 118 58.98) (end 118.02 58.98) (width 0.25) (layer "F.Cu") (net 11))
 (segment (start 124.1002 59.1002) (end 126.8102 59.1002) (width 0.25) (layer "F.Cu") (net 11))
 (segment (start 118.25 58.75) (end 123.75 58.75) (width 0.25) (layer "F.Cu") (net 11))
 (segment (start 124.8998 59.1002) (end 126.8102 59.1002) (width 0.25) (layer "B.Cu") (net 10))
 (segment (start 111.135 65.615) (end 116 60.75) (width 0.25) (layer "B.Cu") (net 10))
 (segment (start 116 60.75) (end 123.25 60.75) (width 0.25) (layer "B.Cu") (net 10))
 (segment (start 95 66.74) (end 96.125 65.615) (width 0.25) (layer "B.Cu") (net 10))
 (segment (start 96.125 65.615) (end 111.135 65.615) (width 0.25) (layer "B.Cu") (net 10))
 (segment (start 123.25 60.75) (end 124.8998 59.1002) (width 0.25) (layer "B.Cu") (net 10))
 (segment (start 110.24 64.2) (end 116.94 57.5) (width 0.25) (layer "F.Cu") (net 9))
 (segment (start 123.25 57.5) (end 124.1898 56.5602) (width 0.25) (layer "F.Cu") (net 9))
 (segment (start 116.94 57.5) (end 123.25 57.5) (width 0.25) (layer "F.Cu") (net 9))
 (segment (start 124.1898 56.5602) (end 126.8102 56.5602) (width 0.25) (layer "F.Cu") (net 9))
 (segment (start 111.345 68.155) (end 112.25 67.25) (width 0.25) (layer "B.Cu") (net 12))
 (segment (start 96.125 68.155) (end 111.345 68.155) (width 0.25) (layer "B.Cu") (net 12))
 (segment (start 112.25 65.75) (end 116.3598 61.6402) (width 0.25) (layer "B.Cu") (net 12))
 (segment (start 112.25 67.25) (end 112.25 65.75) (width 0.25) (layer "B.Cu") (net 12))
 (segment (start 95 69.28) (end 96.125 68.155) (width 0.25) (layer "B.Cu") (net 12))
 (segment (start 116.3598 61.6402) (end 126.8102 61.6402) (width 0.25) (layer "B.Cu") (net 12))
 (segment (start 115.4 56.5) (end 121 56.5) (width 0.25) (layer "F.Cu") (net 7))
 (segment (start 123.4798 54.0202) (end 126.8102 54.0202) (width 0.25) (layer "F.Cu") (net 7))
 (segment (start 121 56.5) (end 123.4798 54.0202) (width 0.25) (layer "F.Cu") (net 7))
 (segment (start 110.24 61.66) (end 115.4 56.5) (width 0.25) (layer "F.Cu") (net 7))
 (segment (start 119.75 74.25) (end 123.25 70.75) (width 0.25) (layer "B.Cu") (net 14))
 (segment (start 96.125 70.695) (end 111.945 70.695) (width 0.25) (layer "B.Cu") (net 14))
 (segment (start 115.5 74.25) (end 119.75 74.25) (width 0.25) (layer "B.Cu") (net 14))
 (segment (start 95 71.82) (end 96.125 70.695) (width 0.25) (layer "B.Cu") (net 14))
 (segment (start 123.25 70.75) (end 123.25 66) (width 0.25) (layer "B.Cu") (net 14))
 (segment (start 111.945 70.695) (end 115.5 74.25) (width 0.25) (layer "B.Cu") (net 14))
 (segment (start 125.0698 64.1802) (end 126.8102 64.1802) (width 0.25) (layer "B.Cu") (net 14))
 (segment (start 123.25 66) (end 125.0698 64.1802) (width 0.25) (layer "B.Cu") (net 14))
 (segment (start 120.25 55.5) (end 124.2698 51.4802) (width 0.25) (layer "F.Cu") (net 5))
 (segment (start 115.25 55.5) (end 120.25 55.5) (width 0.25) (layer "F.Cu") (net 5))
 (segment (start 111.63 59.12) (end 115.25 55.5) (width 0.25) (layer "F.Cu") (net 5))
 (segment (start 110.24 59.12) (end 111.63 59.12) (width 0.25) (layer "F.Cu") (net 5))
 (segment (start 124.2698 51.4802) (end 126.8102 51.4802) (width 0.25) (layer "F.Cu") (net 5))
 (segment (start 96.125 73.235) (end 112.735 73.235) (width 0.25) (layer "B.Cu") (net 16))
 (segment (start 120.5 75) (end 124.25 71.25) (width 0.25) (layer "B.Cu") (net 16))
 (segment (start 95 74.36) (end 96.125 73.235) (width 0.25) (layer "B.Cu") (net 16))
 (segment (start 125.7798 66.7202) (end 126.8102 66.7202) (width 0.25) (layer "B.Cu") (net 16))
 (segment (start 124.25 68.25) (end 125.7798 66.7202) (width 0.25) (layer "B.Cu") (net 16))
 (segment (start 124.25 71.25) (end 124.25 68.25) (width 0.25) (layer "B.Cu") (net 16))
 (segment (start 114.5 75) (end 120.5 75) (width 0.25) (layer "B.Cu") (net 16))
 (segment (start 112.735 73.235) (end 114.5 75) (width 0.25) (layer "B.Cu") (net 16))
 (segment (start 125 69.75) (end 125.4898 69.2602) (width 0.25) (layer "B.Cu") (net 18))
 (segment (start 125 71.5) (end 125 69.75) (width 0.25) (layer "B.Cu") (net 18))
 (segment (start 118 76.5) (end 120 76.5) (width 0.25) (layer "B.Cu") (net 18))
 (segment (start 96.125 75.775) (end 117.275 75.775) (width 0.25) (layer "B.Cu") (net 18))
 (segment (start 120 76.5) (end 125 71.5) (width 0.25) (layer "B.Cu") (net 18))
 (segment (start 125.4898 69.2602) (end 126.8102 69.2602) (width 0.25) (layer "B.Cu") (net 18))
 (segment (start 95 76.9) (end 96.125 75.775) (width 0.25) (layer "B.Cu") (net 18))
 (segment (start 117.275 75.775) (end 118 76.5) (width 0.25) (layer "B.Cu") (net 18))
 (segment (start 125.9498 71.8002) (end 126.8102 71.8002) (width 0.25) (layer "B.Cu") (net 20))
 (segment (start 117.185 78.315) (end 118 77.5) (width 0.25) (layer "B.Cu") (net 20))
 (segment (start 118 77.5) (end 120.25 77.5) (width 0.25) (layer "B.Cu") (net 20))
 (segment (start 95 79.44) (end 96.125 78.315) (width 0.25) (layer "B.Cu") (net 20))
 (segment (start 96.125 78.315) (end 117.185 78.315) (width 0.25) (layer "B.Cu") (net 20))
 (segment (start 120.25 77.5) (end 125.9498 71.8002) (width 0.25) (layer "B.Cu") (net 20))
 (segment (start 115.645 80.855) (end 96.125 80.855) (width 0.25) (layer "B.Cu") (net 22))
 (segment (start 125.1598 74.3402) (end 121 78.5) (width 0.25) (layer "B.Cu") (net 22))
 (segment (start 126.8102 74.3402) (end 125.1598 74.3402) (width 0.25) (layer "B.Cu") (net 22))
 (segment (start 118 78.5) (end 115.645 80.855) (width 0.25) (layer "B.Cu") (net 22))
 (segment (start 121 78.5) (end 118 78.5) (width 0.25) (layer "B.Cu") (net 22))
 (segment (start 96.125 80.855) (end 95 81.98) (width 0.25) (layer "B.Cu") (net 22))
 (segment (start 98.99 47.5) (end 97.25 47.5) (width 0.25) (layer "F.Cu") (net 30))
 (via (at 97.25 47.5) (size 0.8) (drill 0.4) (layers "F.Cu" "B.Cu") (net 30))
 (segment (start 120.5 91) (end 124.4598 87.0402) (width 0.25) (layer "B.Cu") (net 30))
 (segment (start 97.25 47.5) (end 91.25 47.5) (width 0.25) (layer "B.Cu") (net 30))
 (segment (start 124.4598 87.0402) (end 126.8102 87.0402) (width 0.25) (layer "B.Cu") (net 30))
 (segment (start 90 48.75) (end 90 88.25) (width 0.25) (layer "B.Cu") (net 30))
 (segment (start 91.25 47.5) (end 90 48.75) (width 0.25) (layer "B.Cu") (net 30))
 (segment (start 90 88.25) (end 92.75 91) (width 0.25) (layer "B.Cu") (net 30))
 (segment (start 92.75 91) (end 120.5 91) (width 0.25) (layer "B.Cu") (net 30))
 (segment (start 107.25 56.5) (end 107.25 57.75) (width 0.25) (layer "F.Cu") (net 28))
 (segment (start 107.25 57.75) (end 107.25 88.5) (width 0.25) (layer "F.Cu") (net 28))
 (via (at 107.25 56.5) (size 0.8) (drill 0.4) (layers "F.Cu" "B.Cu") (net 28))
 (via (at 107.25 88.5) (size 0.8) (drill 0.4) (layers "F.Cu" "B.Cu") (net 28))
 (segment (start 124.7498 84.5002) (end 126.8102 84.5002) (width 0.25) (layer "B.Cu") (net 28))
 (segment (start 122.75 86.5) (end 124.7498 84.5002) (width 0.25) (layer "B.Cu") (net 28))
 (segment (start 110.24 56.58) (end 107.33 56.58) (width 0.25) (layer "B.Cu") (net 28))
 (segment (start 109 90.25) (end 120 90.25) (width 0.25) (layer "B.Cu") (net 28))
 (segment (start 107.33 56.58) (end 107.25 56.5) (width 0.25) (layer "B.Cu") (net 28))
 (segment (start 122.75 87.5) (end 122.75 86.5) (width 0.25) (layer "B.Cu") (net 28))
 (segment (start 120 90.25) (end 122.75 87.5) (width 0.25) (layer "B.Cu") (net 28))
 (segment (start 107.25 88.5) (end 109 90.25) (width 0.25) (layer "B.Cu") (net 28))
 (segment (start 105.21 50.71) (end 108.54 54.04) (width 0.25) (layer "F.Cu") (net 34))
 (segment (start 108.54 54.04) (end 110.24 54.04) (width 0.25) (layer "F.Cu") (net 34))
 (segment (start 100.01 47.5) (end 105.21 47.5) (width 0.25) (layer "F.Cu") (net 34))
 (segment (start 105.21 47.5) (end 105.21 50.71) (width 0.25) (layer "F.Cu") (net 34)))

